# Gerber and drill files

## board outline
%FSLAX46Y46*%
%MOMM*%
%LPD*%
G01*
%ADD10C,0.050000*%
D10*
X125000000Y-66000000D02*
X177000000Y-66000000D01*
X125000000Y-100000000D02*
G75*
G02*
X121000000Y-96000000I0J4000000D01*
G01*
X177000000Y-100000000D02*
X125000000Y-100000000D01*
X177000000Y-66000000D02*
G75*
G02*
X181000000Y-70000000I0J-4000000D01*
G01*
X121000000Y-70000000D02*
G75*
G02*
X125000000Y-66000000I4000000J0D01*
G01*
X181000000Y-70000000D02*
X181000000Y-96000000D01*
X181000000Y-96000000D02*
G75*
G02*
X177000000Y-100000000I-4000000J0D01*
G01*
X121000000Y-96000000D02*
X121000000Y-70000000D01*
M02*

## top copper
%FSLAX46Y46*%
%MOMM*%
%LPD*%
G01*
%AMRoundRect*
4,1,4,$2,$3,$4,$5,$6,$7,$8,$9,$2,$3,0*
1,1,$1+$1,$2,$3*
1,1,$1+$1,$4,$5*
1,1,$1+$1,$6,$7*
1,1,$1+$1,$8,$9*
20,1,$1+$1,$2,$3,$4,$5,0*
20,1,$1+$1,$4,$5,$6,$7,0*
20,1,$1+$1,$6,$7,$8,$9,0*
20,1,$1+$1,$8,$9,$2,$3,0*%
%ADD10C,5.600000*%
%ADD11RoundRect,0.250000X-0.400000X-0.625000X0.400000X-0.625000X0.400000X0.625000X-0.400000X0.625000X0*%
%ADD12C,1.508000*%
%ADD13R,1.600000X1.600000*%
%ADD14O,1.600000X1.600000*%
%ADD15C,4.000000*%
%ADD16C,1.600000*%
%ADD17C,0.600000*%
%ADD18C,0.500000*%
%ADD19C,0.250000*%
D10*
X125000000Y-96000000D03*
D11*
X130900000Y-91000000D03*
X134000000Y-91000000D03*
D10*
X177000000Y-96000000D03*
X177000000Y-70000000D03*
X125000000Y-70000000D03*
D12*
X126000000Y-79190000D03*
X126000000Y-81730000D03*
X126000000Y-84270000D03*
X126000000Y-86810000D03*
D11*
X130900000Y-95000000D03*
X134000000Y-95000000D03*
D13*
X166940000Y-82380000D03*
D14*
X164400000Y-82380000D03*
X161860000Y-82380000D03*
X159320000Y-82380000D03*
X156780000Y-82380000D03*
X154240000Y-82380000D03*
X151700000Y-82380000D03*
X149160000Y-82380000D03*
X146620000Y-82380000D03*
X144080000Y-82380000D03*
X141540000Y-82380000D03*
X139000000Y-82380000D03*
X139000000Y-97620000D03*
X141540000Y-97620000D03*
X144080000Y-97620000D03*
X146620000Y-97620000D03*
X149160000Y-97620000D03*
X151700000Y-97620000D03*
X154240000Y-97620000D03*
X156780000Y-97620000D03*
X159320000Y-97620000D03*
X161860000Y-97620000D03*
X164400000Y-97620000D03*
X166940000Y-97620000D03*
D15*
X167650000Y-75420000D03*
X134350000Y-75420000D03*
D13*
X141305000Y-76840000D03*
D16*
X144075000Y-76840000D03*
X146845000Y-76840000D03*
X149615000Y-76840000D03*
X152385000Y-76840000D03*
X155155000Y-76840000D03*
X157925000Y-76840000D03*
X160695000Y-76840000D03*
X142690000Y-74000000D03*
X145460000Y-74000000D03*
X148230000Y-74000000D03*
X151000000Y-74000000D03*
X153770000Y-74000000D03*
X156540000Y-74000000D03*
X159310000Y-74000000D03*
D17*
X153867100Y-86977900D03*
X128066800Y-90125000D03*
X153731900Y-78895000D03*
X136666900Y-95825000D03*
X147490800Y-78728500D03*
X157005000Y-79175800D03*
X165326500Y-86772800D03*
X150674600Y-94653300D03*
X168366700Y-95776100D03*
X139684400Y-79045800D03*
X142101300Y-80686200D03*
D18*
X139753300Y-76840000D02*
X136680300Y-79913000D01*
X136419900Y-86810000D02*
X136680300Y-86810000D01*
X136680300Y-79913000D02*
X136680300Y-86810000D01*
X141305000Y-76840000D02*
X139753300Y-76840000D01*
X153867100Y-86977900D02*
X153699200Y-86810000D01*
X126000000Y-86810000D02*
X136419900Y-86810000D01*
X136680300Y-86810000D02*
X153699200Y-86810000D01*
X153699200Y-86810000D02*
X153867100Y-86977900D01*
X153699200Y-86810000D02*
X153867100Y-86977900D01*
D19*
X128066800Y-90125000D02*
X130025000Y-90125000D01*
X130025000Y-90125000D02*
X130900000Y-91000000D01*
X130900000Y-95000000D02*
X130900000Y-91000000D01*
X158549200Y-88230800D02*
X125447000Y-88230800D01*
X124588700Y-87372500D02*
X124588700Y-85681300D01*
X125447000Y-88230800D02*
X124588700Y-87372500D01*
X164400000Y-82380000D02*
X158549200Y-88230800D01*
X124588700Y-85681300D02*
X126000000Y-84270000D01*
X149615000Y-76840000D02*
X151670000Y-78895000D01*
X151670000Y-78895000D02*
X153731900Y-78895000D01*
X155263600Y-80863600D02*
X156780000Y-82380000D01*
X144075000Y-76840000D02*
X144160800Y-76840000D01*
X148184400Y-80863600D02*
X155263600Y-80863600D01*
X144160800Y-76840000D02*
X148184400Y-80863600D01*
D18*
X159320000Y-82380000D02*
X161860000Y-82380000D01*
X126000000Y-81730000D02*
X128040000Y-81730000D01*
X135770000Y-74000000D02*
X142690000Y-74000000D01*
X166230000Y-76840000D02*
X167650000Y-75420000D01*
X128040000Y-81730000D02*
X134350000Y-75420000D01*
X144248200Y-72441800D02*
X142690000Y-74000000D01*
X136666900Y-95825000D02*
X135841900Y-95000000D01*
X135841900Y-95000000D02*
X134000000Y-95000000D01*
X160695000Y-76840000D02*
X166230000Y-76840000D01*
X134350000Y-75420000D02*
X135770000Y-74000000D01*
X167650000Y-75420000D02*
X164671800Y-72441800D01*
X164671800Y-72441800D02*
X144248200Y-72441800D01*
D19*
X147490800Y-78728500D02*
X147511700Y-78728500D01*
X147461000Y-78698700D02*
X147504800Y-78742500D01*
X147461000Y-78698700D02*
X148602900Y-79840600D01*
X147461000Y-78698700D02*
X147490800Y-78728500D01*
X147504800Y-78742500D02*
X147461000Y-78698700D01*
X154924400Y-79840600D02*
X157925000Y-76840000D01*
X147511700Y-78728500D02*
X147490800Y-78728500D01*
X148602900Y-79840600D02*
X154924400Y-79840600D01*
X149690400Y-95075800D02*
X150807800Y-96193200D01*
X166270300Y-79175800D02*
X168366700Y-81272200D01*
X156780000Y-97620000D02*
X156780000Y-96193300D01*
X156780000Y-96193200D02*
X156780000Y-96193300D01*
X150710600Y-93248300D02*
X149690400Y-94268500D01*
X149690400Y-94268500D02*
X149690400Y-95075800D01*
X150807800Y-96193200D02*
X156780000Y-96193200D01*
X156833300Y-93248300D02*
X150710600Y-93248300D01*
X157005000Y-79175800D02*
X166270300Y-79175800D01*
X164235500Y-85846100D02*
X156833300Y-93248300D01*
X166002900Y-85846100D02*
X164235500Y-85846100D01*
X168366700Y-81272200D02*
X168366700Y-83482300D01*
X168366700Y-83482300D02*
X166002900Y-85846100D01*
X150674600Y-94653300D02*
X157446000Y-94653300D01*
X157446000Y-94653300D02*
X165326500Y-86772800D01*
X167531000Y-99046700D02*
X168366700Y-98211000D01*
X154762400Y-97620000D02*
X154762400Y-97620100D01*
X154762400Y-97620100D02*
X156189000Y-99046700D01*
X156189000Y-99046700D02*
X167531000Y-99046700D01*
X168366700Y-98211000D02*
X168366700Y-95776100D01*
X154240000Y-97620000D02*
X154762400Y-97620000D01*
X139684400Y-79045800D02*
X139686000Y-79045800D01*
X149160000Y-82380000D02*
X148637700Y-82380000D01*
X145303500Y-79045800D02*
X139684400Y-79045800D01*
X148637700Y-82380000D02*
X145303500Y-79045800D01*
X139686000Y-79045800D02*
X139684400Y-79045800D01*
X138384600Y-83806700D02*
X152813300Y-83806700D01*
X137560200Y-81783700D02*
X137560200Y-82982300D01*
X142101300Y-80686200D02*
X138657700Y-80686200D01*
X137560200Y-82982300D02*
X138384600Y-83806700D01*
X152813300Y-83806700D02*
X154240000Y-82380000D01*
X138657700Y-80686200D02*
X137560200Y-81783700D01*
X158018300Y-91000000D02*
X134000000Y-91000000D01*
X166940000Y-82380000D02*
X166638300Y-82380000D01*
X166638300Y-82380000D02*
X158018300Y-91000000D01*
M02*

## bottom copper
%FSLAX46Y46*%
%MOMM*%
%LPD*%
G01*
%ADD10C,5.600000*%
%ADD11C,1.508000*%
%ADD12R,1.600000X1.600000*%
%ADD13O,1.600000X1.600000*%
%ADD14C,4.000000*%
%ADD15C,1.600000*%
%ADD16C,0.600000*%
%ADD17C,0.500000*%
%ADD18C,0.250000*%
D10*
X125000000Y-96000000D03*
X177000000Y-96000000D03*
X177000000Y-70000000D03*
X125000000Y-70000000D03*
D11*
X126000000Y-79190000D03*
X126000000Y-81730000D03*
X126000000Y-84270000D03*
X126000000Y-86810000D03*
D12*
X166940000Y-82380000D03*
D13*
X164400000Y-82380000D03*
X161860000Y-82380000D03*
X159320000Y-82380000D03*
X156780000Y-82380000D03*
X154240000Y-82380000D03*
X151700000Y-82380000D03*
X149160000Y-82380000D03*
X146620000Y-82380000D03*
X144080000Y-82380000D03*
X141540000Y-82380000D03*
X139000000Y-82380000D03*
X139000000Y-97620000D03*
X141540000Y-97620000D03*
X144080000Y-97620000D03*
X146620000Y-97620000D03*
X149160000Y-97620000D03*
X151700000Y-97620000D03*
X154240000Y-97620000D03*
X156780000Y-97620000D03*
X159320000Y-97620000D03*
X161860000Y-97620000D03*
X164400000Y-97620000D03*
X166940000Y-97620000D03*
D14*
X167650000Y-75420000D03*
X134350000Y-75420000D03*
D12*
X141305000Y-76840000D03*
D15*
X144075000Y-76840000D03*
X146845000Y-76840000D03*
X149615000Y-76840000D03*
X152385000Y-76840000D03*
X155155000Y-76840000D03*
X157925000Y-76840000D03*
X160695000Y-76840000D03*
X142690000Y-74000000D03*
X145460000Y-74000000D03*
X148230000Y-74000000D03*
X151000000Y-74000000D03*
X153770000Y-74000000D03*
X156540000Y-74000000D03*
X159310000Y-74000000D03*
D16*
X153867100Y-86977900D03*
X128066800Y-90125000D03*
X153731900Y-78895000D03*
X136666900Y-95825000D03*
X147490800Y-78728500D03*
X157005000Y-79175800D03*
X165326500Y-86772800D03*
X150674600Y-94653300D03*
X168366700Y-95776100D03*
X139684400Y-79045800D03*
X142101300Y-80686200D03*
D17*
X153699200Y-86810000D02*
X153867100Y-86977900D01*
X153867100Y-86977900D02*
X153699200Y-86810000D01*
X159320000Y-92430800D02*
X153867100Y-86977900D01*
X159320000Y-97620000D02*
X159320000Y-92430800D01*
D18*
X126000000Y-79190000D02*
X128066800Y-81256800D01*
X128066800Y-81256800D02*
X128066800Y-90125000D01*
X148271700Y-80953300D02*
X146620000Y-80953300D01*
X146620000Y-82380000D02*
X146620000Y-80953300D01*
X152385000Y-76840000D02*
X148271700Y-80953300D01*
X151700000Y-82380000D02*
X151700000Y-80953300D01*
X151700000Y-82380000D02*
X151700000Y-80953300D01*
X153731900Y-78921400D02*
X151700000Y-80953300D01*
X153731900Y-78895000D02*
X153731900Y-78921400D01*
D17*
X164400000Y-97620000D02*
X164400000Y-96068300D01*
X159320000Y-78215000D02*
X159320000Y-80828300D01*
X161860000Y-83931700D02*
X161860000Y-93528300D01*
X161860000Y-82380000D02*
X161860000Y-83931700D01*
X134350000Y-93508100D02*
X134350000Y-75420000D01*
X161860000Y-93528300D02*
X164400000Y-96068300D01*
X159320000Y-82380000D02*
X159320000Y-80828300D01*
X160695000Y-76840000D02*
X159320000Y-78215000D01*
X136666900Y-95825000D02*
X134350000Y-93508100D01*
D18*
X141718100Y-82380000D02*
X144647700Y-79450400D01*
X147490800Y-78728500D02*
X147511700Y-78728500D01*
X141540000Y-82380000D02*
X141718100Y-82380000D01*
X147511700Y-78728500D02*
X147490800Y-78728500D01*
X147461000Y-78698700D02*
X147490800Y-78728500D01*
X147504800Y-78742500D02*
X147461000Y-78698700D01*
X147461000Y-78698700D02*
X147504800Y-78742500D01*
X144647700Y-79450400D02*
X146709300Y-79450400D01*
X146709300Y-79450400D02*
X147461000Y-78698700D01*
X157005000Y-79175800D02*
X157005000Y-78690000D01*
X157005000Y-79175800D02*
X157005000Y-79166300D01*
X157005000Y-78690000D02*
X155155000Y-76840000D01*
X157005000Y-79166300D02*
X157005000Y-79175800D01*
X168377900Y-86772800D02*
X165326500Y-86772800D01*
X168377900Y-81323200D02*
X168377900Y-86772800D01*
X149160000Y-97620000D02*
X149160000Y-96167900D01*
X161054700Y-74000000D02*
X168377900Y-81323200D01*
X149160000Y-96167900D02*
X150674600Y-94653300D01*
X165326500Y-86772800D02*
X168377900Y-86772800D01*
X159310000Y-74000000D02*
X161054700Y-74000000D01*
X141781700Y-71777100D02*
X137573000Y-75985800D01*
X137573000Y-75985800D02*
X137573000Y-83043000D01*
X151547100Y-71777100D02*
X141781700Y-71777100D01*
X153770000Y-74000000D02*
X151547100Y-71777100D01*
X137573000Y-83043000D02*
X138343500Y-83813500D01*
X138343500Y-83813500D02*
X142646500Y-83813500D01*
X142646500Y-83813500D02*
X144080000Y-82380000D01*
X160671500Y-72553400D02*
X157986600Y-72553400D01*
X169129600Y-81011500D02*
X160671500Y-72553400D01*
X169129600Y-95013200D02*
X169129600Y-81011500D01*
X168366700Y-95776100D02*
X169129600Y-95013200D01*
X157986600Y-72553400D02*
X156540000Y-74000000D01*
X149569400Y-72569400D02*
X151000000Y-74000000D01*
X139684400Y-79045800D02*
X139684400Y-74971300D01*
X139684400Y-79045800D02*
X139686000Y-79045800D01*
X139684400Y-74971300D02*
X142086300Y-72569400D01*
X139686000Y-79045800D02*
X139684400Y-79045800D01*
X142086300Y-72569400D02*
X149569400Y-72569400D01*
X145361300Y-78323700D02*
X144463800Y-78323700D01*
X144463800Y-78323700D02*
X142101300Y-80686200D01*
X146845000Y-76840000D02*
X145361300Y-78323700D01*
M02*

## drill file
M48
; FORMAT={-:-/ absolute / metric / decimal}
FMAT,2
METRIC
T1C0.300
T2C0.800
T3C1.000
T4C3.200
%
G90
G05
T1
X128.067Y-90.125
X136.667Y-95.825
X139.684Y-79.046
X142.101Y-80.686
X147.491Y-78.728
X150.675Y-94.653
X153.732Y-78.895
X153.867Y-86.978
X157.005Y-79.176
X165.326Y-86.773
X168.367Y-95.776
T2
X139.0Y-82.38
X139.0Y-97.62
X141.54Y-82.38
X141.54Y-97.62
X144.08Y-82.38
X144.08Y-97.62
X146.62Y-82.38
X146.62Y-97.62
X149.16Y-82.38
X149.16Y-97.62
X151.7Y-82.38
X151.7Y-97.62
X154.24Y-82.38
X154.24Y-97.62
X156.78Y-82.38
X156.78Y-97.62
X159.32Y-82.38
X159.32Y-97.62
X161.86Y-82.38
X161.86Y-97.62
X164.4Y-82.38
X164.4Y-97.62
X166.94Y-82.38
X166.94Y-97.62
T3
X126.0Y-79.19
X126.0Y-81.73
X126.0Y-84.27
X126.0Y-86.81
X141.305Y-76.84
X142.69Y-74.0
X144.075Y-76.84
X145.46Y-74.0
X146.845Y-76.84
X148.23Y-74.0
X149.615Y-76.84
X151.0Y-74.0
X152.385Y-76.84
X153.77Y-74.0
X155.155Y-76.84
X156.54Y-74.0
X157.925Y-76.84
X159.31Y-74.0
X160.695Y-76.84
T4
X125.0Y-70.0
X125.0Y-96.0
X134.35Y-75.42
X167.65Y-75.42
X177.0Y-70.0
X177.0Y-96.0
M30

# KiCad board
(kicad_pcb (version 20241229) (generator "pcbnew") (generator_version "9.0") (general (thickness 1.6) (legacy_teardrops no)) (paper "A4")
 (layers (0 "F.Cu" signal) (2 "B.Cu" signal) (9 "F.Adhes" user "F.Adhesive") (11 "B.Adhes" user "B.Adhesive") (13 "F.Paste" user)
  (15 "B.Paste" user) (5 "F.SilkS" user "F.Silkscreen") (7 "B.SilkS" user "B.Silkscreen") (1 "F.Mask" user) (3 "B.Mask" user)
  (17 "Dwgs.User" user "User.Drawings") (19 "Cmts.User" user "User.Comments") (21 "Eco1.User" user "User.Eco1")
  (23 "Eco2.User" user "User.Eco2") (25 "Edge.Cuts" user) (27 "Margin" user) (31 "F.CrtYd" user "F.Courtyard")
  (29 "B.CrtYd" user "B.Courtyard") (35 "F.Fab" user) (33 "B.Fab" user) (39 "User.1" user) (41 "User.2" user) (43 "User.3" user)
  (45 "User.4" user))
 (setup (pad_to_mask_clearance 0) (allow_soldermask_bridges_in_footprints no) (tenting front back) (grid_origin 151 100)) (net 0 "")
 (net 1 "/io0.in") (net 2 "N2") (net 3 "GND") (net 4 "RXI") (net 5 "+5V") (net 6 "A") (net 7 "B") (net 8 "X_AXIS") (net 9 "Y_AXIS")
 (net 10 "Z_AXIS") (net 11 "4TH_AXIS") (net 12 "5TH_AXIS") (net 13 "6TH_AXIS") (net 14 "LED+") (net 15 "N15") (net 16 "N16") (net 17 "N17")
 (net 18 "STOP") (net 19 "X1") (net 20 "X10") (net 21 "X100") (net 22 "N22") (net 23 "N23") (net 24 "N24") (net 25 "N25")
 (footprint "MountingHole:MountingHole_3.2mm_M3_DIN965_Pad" (layer "F.Cu") (at 125 96)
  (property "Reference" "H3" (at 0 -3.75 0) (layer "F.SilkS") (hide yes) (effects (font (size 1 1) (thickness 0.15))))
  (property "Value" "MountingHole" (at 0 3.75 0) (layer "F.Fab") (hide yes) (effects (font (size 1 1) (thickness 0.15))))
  (pad "1" thru_hole circle (at 0 0) (size 5.6 5.6) (drill 3.2) (layers "*.Cu" "*.Mask") (remove_unused_layers no) (zone_connect 2)))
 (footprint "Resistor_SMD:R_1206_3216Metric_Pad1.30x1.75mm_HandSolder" (layer "F.Cu") (at 132.45 91)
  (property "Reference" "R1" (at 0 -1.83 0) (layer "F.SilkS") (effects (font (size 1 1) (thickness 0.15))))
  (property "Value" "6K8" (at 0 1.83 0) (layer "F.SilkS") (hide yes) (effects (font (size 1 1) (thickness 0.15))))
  (pad "1" smd roundrect (at -1.55 0) (size 1.3 1.75) (layers "F.Cu" "F.Mask" "F.Paste") (roundrect_rratio 0.192308) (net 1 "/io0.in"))
  (pad "2" smd roundrect (at 1.55 0) (size 1.3 1.75) (layers "F.Cu" "F.Mask" "F.Paste") (roundrect_rratio 0.192308) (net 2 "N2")))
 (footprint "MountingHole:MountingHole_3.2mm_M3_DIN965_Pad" (layer "F.Cu") (at 177 96)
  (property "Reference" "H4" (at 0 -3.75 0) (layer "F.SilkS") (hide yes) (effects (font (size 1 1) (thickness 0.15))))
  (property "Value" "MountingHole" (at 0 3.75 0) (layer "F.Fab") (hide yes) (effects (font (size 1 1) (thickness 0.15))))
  (pad "1" thru_hole circle (at 0 0) (size 5.6 5.6) (drill 3.2) (layers "*.Cu" "*.Mask") (remove_unused_layers no) (zone_connect 2)))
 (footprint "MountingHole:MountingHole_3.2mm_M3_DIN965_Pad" (layer "F.Cu") (at 177 70)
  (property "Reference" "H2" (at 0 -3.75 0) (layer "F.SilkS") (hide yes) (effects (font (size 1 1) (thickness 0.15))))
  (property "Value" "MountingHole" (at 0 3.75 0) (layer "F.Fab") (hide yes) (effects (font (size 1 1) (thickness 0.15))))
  (pad "1" thru_hole circle (at 0 0) (size 5.6 5.6) (drill 3.2) (layers "*.Cu" "*.Mask") (remove_unused_layers no) (zone_connect 2)))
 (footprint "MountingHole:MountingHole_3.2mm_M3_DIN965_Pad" (layer "F.Cu") (at 125 70)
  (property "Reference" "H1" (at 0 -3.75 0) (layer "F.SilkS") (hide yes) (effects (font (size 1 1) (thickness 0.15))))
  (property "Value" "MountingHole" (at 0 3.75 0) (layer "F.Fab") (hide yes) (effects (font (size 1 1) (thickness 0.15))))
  (pad "1" thru_hole circle (at 0 0) (size 5.6 5.6) (drill 3.2) (layers "*.Cu" "*.Mask") (remove_unused_layers no) (zone_connect 2)))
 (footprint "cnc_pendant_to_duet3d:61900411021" (layer "F.Cu") (at 122.65 83 -90)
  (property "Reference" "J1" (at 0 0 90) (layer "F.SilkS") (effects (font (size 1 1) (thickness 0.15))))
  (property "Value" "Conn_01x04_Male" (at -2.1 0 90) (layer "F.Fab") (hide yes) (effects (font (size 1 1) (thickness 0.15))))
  (pad "1" thru_hole circle (at -3.81 -3.35 270) (size 1.508 1.508) (drill 1) (layers "*.Cu" "*.Mask") (remove_unused_layers no)
   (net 1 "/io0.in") (solder_mask_margin 0.102))
  (pad "2" thru_hole circle (at -1.27 -3.35 270) (size 1.508 1.508) (drill 1) (layers "*.Cu" "*.Mask") (remove_unused_layers no)
   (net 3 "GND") (solder_mask_margin 0.102))
  (pad "3" thru_hole circle (at 1.27 -3.35 270) (size 1.508 1.508) (drill 1) (layers "*.Cu" "*.Mask") (remove_unused_layers no)
   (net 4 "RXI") (solder_mask_margin 0.102))
  (pad "4" thru_hole circle (at 3.81 -3.35 270) (size 1.508 1.508) (drill 1) (layers "*.Cu" "*.Mask") (remove_unused_layers no)
   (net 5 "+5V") (solder_mask_margin 0.102)))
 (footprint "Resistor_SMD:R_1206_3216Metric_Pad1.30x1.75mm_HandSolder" (layer "F.Cu") (at 132.45 95)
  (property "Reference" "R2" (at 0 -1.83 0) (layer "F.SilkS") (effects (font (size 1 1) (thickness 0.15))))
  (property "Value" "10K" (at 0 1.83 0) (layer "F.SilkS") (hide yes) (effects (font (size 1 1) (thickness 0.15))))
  (pad "1" smd roundrect (at -1.55 0) (size 1.3 1.75) (layers "F.Cu" "F.Mask" "F.Paste") (roundrect_rratio 0.192308) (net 1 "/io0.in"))
  (pad "2" smd roundrect (at 1.55 0) (size 1.3 1.75) (layers "F.Cu" "F.Mask" "F.Paste") (roundrect_rratio 0.192308) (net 3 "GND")))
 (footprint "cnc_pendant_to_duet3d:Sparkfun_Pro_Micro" (layer "F.Cu") (at 139 97.62 90)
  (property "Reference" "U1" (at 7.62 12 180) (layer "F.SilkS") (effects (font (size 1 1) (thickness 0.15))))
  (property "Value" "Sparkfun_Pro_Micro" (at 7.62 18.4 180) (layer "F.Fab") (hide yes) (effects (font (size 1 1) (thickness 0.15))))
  (pad "1" thru_hole rect (at 15.24 27.94 90) (size 1.6 1.6) (drill 0.8) (layers "*.Cu" "*.Mask") (remove_unused_layers no) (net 2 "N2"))
  (pad "2" thru_hole oval (at 15.24 25.4 90) (size 1.6 1.6) (drill 0.8) (layers "*.Cu" "*.Mask") (remove_unused_layers no) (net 4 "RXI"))
  (pad "3" thru_hole oval (at 15.24 22.86 90) (size 1.6 1.6) (drill 0.8) (layers "*.Cu" "*.Mask") (remove_unused_layers no) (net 3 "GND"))
  (pad "4" thru_hole oval (at 15.24 20.32 90) (size 1.6 1.6) (drill 0.8) (layers "*.Cu" "*.Mask") (remove_unused_layers no) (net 3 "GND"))
  (pad "5" thru_hole oval (at 15.24 17.78 90) (size 1.6 1.6) (drill 0.8) (layers "*.Cu" "*.Mask") (remove_unused_layers no) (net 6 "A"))
  (pad "6" thru_hole oval (at 15.24 15.24 90) (size 1.6 1.6) (drill 0.8) (layers "*.Cu" "*.Mask") (remove_unused_layers no) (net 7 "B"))
  (pad "7" thru_hole oval (at 15.24 12.7 90) (size 1.6 1.6) (drill 0.8) (layers "*.Cu" "*.Mask") (remove_unused_layers no) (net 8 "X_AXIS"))
  (pad "8" thru_hole oval (at 15.24 10.16 90) (size 1.6 1.6) (drill 0.8) (layers "*.Cu" "*.Mask") (remove_unused_layers no) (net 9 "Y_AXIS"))
  (pad "9" thru_hole oval (at 15.24 7.62 90) (size 1.6 1.6) (drill 0.8) (layers "*.Cu" "*.Mask") (remove_unused_layers no) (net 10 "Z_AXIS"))
  (pad "10" thru_hole oval (at 15.24 5.08 90) (size 1.6 1.6) (drill 0.8) (layers "*.Cu" "*.Mask") (remove_unused_layers no)
   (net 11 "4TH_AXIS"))
  (pad "11" thru_hole oval (at 15.24 2.54 90) (size 1.6 1.6) (drill 0.8) (layers "*.Cu" "*.Mask") (remove_unused_layers no)
   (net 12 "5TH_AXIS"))
  (pad "12" thru_hole oval (at 15.24 0 90) (size 1.6 1.6) (drill 0.8) (layers "*.Cu" "*.Mask") (remove_unused_layers no) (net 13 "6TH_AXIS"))
  (pad "13" thru_hole oval (at 0 0 90) (size 1.6 1.6) (drill 0.8) (layers "*.Cu" "*.Mask") (remove_unused_layers no) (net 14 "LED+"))
  (pad "14" thru_hole oval (at 0 2.54 90) (size 1.6 1.6) (drill 0.8) (layers "*.Cu" "*.Mask") (remove_unused_layers no) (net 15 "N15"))
  (pad "15" thru_hole oval (at 0 5.08 90) (size 1.6 1.6) (drill 0.8) (layers "*.Cu" "*.Mask") (remove_unused_layers no) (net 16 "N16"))
  (pad "16" thru_hole oval (at 0 7.62 90) (size 1.6 1.6) (drill 0.8) (layers "*.Cu" "*.Mask") (remove_unused_layers no) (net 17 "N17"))
  (pad "17" thru_hole oval (at 0 10.16 90) (size 1.6 1.6) (drill 0.8) (layers "*.Cu" "*.Mask") (remove_unused_layers no) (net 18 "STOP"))
  (pad "18" thru_hole oval (at 0 12.7 90) (size 1.6 1.6) (drill 0.8) (layers "*.Cu" "*.Mask") (remove_unused_layers no) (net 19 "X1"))
  (pad "19" thru_hole oval (at 0 15.24 90) (size 1.6 1.6) (drill 0.8) (layers "*.Cu" "*.Mask") (remove_unused_layers no) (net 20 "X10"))
  (pad "20" thru_hole oval (at 0 17.78 90) (size 1.6 1.6) (drill 0.8) (layers "*.Cu" "*.Mask") (remove_unused_layers no) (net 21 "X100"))
  (pad "21" thru_hole oval (at 0 20.32 90) (size 1.6 1.6) (drill 0.8) (layers "*.Cu" "*.Mask") (remove_unused_layers no) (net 5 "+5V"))
  (pad "22" thru_hole oval (at 0 22.86 90) (size 1.6 1.6) (drill 0.8) (layers "*.Cu" "*.Mask") (remove_unused_layers no) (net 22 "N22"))
  (pad "23" thru_hole oval (at 0 25.4 90) (size 1.6 1.6) (drill 0.8) (layers "*.Cu" "*.Mask") (remove_unused_layers no) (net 3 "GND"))
  (pad "24" thru_hole oval (at 0 27.94 90) (size 1.6 1.6) (drill 0.8) (layers "*.Cu" "*.Mask") (remove_unused_layers no) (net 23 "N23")))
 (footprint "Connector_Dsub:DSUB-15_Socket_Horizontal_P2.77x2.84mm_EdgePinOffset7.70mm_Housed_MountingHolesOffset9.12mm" (layer "F.Cu")
  (at 141.305 76.84 180)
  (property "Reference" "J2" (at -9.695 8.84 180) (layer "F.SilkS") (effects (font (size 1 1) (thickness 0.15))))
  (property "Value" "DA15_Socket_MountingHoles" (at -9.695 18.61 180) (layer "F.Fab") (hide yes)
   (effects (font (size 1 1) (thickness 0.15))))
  (pad "0" thru_hole circle (at -26.345 1.42 180) (size 4 4) (drill 3.2) (layers "*.Cu" "*.Mask") (remove_unused_layers no) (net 3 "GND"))
  (pad "0" thru_hole circle (at 6.955 1.42 180) (size 4 4) (drill 3.2) (layers "*.Cu" "*.Mask") (remove_unused_layers no) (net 3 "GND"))
  (pad "1" thru_hole rect (at 0 0 180) (size 1.6 1.6) (drill 1) (layers "*.Cu" "*.Mask") (remove_unused_layers no) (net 5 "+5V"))
  (pad "2" thru_hole circle (at -2.77 0 180) (size 1.6 1.6) (drill 1) (layers "*.Cu" "*.Mask") (remove_unused_layers no) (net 6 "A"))
  (pad "3" thru_hole circle (at -5.54 0 180) (size 1.6 1.6) (drill 1) (layers "*.Cu" "*.Mask") (remove_unused_layers no) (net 7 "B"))
  (pad "4" thru_hole circle (at -8.31 0 180) (size 1.6 1.6) (drill 1) (layers "*.Cu" "*.Mask") (remove_unused_layers no) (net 8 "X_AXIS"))
  (pad "5" thru_hole circle (at -11.08 0 180) (size 1.6 1.6) (drill 1) (layers "*.Cu" "*.Mask") (remove_unused_layers no) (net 10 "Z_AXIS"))
  (pad "6" thru_hole circle (at -13.85 0 180) (size 1.6 1.6) (drill 1) (layers "*.Cu" "*.Mask") (remove_unused_layers no) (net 21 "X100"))
  (pad "7" thru_hole circle (at -16.62 0 180) (size 1.6 1.6) (drill 1) (layers "*.Cu" "*.Mask") (remove_unused_layers no)
   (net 12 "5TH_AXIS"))
  (pad "8" thru_hole circle (at -19.39 0 180) (size 1.6 1.6) (drill 1) (layers "*.Cu" "*.Mask") (remove_unused_layers no) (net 3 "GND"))
  (pad "9" thru_hole circle (at -1.385 2.84 180) (size 1.6 1.6) (drill 1) (layers "*.Cu" "*.Mask") (remove_unused_layers no) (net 3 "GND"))
  (pad "10" thru_hole circle (at -4.155 2.84 180) (size 1.6 1.6) (drill 1) (layers "*.Cu" "*.Mask") (remove_unused_layers no) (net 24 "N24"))
  (pad "11" thru_hole circle (at -6.925 2.84 180) (size 1.6 1.6) (drill 1) (layers "*.Cu" "*.Mask") (remove_unused_layers no) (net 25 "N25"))
  (pad "12" thru_hole circle (at -9.695 2.84 180) (size 1.6 1.6) (drill 1) (layers "*.Cu" "*.Mask") (remove_unused_layers no)
   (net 9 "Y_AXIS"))
  (pad "13" thru_hole circle (at -12.465 2.84 180) (size 1.6 1.6) (drill 1) (layers "*.Cu" "*.Mask") (remove_unused_layers no)
   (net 11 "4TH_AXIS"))
  (pad "14" thru_hole circle (at -15.235 2.84 180) (size 1.6 1.6) (drill 1) (layers "*.Cu" "*.Mask") (remove_unused_layers no)
   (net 20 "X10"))
  (pad "15" thru_hole circle (at -18.005 2.84 180) (size 1.6 1.6) (drill 1) (layers "*.Cu" "*.Mask") (remove_unused_layers no)
   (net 18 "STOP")))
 (gr_line (start 125 66) (end 177 66) (stroke (width 0.05) (type default)) (layer "Edge.Cuts"))
 (gr_arc (start 125 100) (mid 122.171573 98.828427) (end 121 96) (stroke (width 0.05) (type default)) (layer "Edge.Cuts"))
 (gr_line (start 177 100) (end 125 100) (stroke (width 0.05) (type default)) (layer "Edge.Cuts"))
 (gr_arc (start 177 66) (mid 179.828427 67.171573) (end 181 70) (stroke (width 0.05) (type default)) (layer "Edge.Cuts"))
 (gr_arc (start 121 70) (mid 122.171573 67.171573) (end 125 66) (stroke (width 0.05) (type default)) (layer "Edge.Cuts"))
 (gr_line (start 181 70) (end 181 96) (stroke (width 0.05) (type default)) (layer "Edge.Cuts"))
 (gr_arc (start 181 96) (mid 179.828427 98.828427) (end 177 100) (stroke (width 0.05) (type default)) (layer "Edge.Cuts"))
 (gr_line (start 121 96) (end 121 70) (stroke (width 0.05) (type default)) (layer "Edge.Cuts"))
 (segment (start 139.7533 76.84) (end 136.6803 79.913) (width 0.5) (layer "F.Cu") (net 5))
 (segment (start 136.4199 86.81) (end 136.6803 86.81) (width 0.5) (layer "F.Cu") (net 5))
 (segment (start 136.6803 79.913) (end 136.6803 86.81) (width 0.5) (layer "F.Cu") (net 5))
 (segment (start 141.305 76.84) (end 139.7533 76.84) (width 0.5) (layer "F.Cu") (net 5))
 (segment (start 153.8671 86.9779) (end 153.6992 86.81) (width 0.5) (layer "F.Cu") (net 5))
 (segment (start 126 86.81) (end 136.4199 86.81) (width 0.5) (layer "F.Cu") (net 5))
 (segment (start 136.6803 86.81) (end 153.6992 86.81) (width 0.5) (layer "F.Cu") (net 5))
 (segment (start 153.6992 86.81) (end 153.8671 86.9779) (width 0.5) (layer "F.Cu") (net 5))
 (segment (start 153.6992 86.81) (end 153.8671 86.9779) (width 0.5) (layer "F.Cu") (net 5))
 (via (at 153.8671 86.9779) (size 0.6) (drill 0.3) (layers "F.Cu" "B.Cu") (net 5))
 (segment (start 153.6992 86.81) (end 153.8671 86.9779) (width 0.5) (layer "B.Cu") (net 5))
 (segment (start 153.8671 86.9779) (end 153.6992 86.81) (width 0.5) (layer "B.Cu") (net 5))
 (segment (start 159.32 92.4308) (end 153.8671 86.9779) (width 0.5) (layer "B.Cu") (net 5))
 (segment (start 159.32 97.62) (end 159.32 92.4308) (width 0.5) (layer "B.Cu") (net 5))
 (segment (start 128.0668 90.125) (end 130.025 90.125) (width 0.25) (layer "F.Cu") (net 1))
 (segment (start 130.025 90.125) (end 130.9 91) (width 0.25) (layer "F.Cu") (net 1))
 (segment (start 130.9 95) (end 130.9 91) (width 0.25) (layer "F.Cu") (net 1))
 (via (at 128.0668 90.125) (size 0.6) (drill 0.3) (layers "F.Cu" "B.Cu") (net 1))
 (segment (start 126 79.19) (end 128.0668 81.2568) (width 0.25) (layer "B.Cu") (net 1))
 (segment (start 128.0668 81.2568) (end 128.0668 90.125) (width 0.25) (layer "B.Cu") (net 1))
 (segment (start 158.5492 88.2308) (end 125.447 88.2308) (width 0.25) (layer "F.Cu") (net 4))
 (segment (start 124.5887 87.3725) (end 124.5887 85.6813) (width 0.25) (layer "F.Cu") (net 4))
 (segment (start 125.447 88.2308) (end 124.5887 87.3725) (width 0.25) (layer "F.Cu") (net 4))
 (segment (start 164.4 82.38) (end 158.5492 88.2308) (width 0.25) (layer "F.Cu") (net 4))
 (segment (start 124.5887 85.6813) (end 126 84.27) (width 0.25) (layer "F.Cu") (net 4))
 (segment (start 148.2717 80.9533) (end 146.62 80.9533) (width 0.25) (layer "B.Cu") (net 10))
 (segment (start 146.62 82.38) (end 146.62 80.9533) (width 0.25) (layer "B.Cu") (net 10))
 (segment (start 152.385 76.84) (end 148.2717 80.9533) (width 0.25) (layer "B.Cu") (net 10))
 (segment (start 149.615 76.84) (end 151.67 78.895) (width 0.25) (layer "F.Cu") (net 8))
 (segment (start 151.67 78.895) (end 153.7319 78.895) (width 0.25) (layer "F.Cu") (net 8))
 (via (at 153.7319 78.895) (size 0.6) (drill 0.3) (layers "F.Cu" "B.Cu") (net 8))
 (segment (start 151.7 82.38) (end 151.7 80.9533) (width 0.25) (layer "B.Cu") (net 8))
 (segment (start 151.7 82.38) (end 151.7 80.9533) (width 0.25) (layer "B.Cu") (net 8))
 (segment (start 153.7319 78.9214) (end 151.7 80.9533) (width 0.25) (layer "B.Cu") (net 8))
 (segment (start 153.7319 78.895) (end 153.7319 78.9214) (width 0.25) (layer "B.Cu") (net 8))
 (segment (start 155.2636 80.8636) (end 156.78 82.38) (width 0.25) (layer "F.Cu") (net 6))
 (segment (start 144.075 76.84) (end 144.1608 76.84) (width 0.25) (layer "F.Cu") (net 6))
 (segment (start 148.1844 80.8636) (end 155.2636 80.8636) (width 0.25) (layer "F.Cu") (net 6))
 (segment (start 144.1608 76.84) (end 148.1844 80.8636) (width 0.25) (layer "F.Cu") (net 6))
 (segment (start 159.32 82.38) (end 161.86 82.38) (width 0.5) (layer "F.Cu") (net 3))
 (segment (start 126 81.73) (end 128.04 81.73) (width 0.5) (layer "F.Cu") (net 3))
 (segment (start 135.77 74) (end 142.69 74) (width 0.5) (layer "F.Cu") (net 3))
 (segment (start 166.23 76.84) (end 167.65 75.42) (width 0.5) (layer "F.Cu") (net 3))
 (segment (start 128.04 81.73) (end 134.35 75.42) (width 0.5) (layer "F.Cu") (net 3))
 (segment (start 144.2482 72.4418) (end 142.69 74) (width 0.5) (layer "F.Cu") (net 3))
 (segment (start 136.6669 95.825) (end 135.8419 95) (width 0.5) (layer "F.Cu") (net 3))
 (segment (start 135.8419 95) (end 134 95) (width 0.5) (layer "F.Cu") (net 3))
 (segment (start 160.695 76.84) (end 166.23 76.84) (width 0.5) (layer "F.Cu") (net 3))
 (segment (start 134.35 75.42) (end 135.77 74) (width 0.5) (layer "F.Cu") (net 3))
 (segment (start 167.65 75.42) (end 164.6718 72.4418) (width 0.5) (layer "F.Cu") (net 3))
 (segment (start 164.6718 72.4418) (end 144.2482 72.4418) (width 0.5) (layer "F.Cu") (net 3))
 (via (at 136.6669 95.825) (size 0.6) (drill 0.3) (layers "F.Cu" "B.Cu") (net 3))
 (segment (start 164.4 97.62) (end 164.4 96.0683) (width 0.5) (layer "B.Cu") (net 3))
 (segment (start 159.32 78.215) (end 159.32 80.8283) (width 0.5) (layer "B.Cu") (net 3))
 (segment (start 161.86 83.9317) (end 161.86 93.5283) (width 0.5) (layer "B.Cu") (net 3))
 (segment (start 161.86 82.38) (end 161.86 83.9317) (width 0.5) (layer "B.Cu") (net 3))
 (segment (start 134.35 93.5081) (end 134.35 75.42) (width 0.5) (layer "B.Cu") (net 3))
 (segment (start 161.86 93.5283) (end 164.4 96.0683) (width 0.5) (layer "B.Cu") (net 3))
 (segment (start 159.32 82.38) (end 159.32 80.8283) (width 0.5) (layer "B.Cu") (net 3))
 (segment (start 160.695 76.84) (end 159.32 78.215) (width 0.5) (layer "B.Cu") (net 3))
 (segment (start 136.6669 95.825) (end 134.35 93.5081) (width 0.5) (layer "B.Cu") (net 3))
 (segment (start 147.4908 78.7285) (end 147.5117 78.7285) (width 0.25) (layer "F.Cu") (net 12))
 (segment (start 147.461 78.6987) (end 147.5048 78.7425) (width 0.25) (layer "F.Cu") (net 12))
 (segment (start 147.461 78.6987) (end 148.6029 79.8406) (width 0.25) (layer "F.Cu") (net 12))
 (segment (start 147.461 78.6987) (end 147.4908 78.7285) (width 0.25) (layer "F.Cu") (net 12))
 (segment (start 147.5048 78.7425) (end 147.461 78.6987) (width 0.25) (layer "F.Cu") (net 12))
 (segment (start 154.9244 79.8406) (end 157.925 76.84) (width 0.25) (layer "F.Cu") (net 12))
 (segment (start 147.5117 78.7285) (end 147.4908 78.7285) (width 0.25) (layer "F.Cu") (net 12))
 (segment (start 148.6029 79.8406) (end 154.9244 79.8406) (width 0.25) (layer "F.Cu") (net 12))
 (via (at 147.4908 78.7285) (size 0.6) (drill 0.3) (layers "F.Cu" "B.Cu") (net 12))
 (segment (start 141.7181 82.38) (end 144.6477 79.4504) (width 0.25) (layer "B.Cu") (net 12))
 (segment (start 147.4908 78.7285) (end 147.5117 78.7285) (width 0.25) (layer "B.Cu") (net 12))
 (segment (start 141.54 82.38) (end 141.7181 82.38) (width 0.25) (layer "B.Cu") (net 12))
 (segment (start 147.5117 78.7285) (end 147.4908 78.7285) (width 0.25) (layer "B.Cu") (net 12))
 (segment (start 147.461 78.6987) (end 147.4908 78.7285) (width 0.25) (layer "B.Cu") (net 12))
 (segment (start 147.5048 78.7425) (end 147.461 78.6987) (width 0.25) (layer "B.Cu") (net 12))
 (segment (start 147.461 78.6987) (end 147.5048 78.7425) (width 0.25) (layer "B.Cu") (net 12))
 (segment (start 144.6477 79.4504) (end 146.7093 79.4504) (width 0.25) (layer "B.Cu") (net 12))
 (segment (start 146.7093 79.4504) (end 147.461 78.6987) (width 0.25) (layer "B.Cu") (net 12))
 (segment (start 149.6904 95.0758) (end 150.8078 96.1932) (width 0.25) (layer "F.Cu") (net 21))
 (segment (start 166.2703 79.1758) (end 168.3667 81.2722) (width 0.25) (layer "F.Cu") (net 21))
 (segment (start 156.78 97.62) (end 156.78 96.1933) (width 0.25) (layer "F.Cu") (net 21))
 (segment (start 156.78 96.1932) (end 156.78 96.1933) (width 0.25) (layer "F.Cu") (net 21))
 (segment (start 150.7106 93.2483) (end 149.6904 94.2685) (width 0.25) (layer "F.Cu") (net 21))
 (segment (start 149.6904 94.2685) (end 149.6904 95.0758) (width 0.25) (layer "F.Cu") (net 21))
 (segment (start 150.8078 96.1932) (end 156.78 96.1932) (width 0.25) (layer "F.Cu") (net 21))
 (segment (start 156.8333 93.2483) (end 150.7106 93.2483) (width 0.25) (layer "F.Cu") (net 21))
 (segment (start 157.005 79.1758) (end 166.2703 79.1758) (width 0.25) (layer "F.Cu") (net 21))
 (segment (start 164.2355 85.8461) (end 156.8333 93.2483) (width 0.25) (layer "F.Cu") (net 21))
 (segment (start 166.0029 85.8461) (end 164.2355 85.8461) (width 0.25) (layer "F.Cu") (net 21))
 (segment (start 168.3667 81.2722) (end 168.3667 83.4823) (width 0.25) (layer "F.Cu") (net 21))
 (segment (start 168.3667 83.4823) (end 166.0029 85.8461) (width 0.25) (layer "F.Cu") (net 21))
 (via (at 157.005 79.1758) (size 0.6) (drill 0.3) (layers "F.Cu" "B.Cu") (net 21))
 (segment (start 157.005 79.1758) (end 157.005 78.69) (width 0.25) (layer "B.Cu") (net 21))
 (segment (start 157.005 79.1758) (end 157.005 79.1663) (width 0.25) (layer "B.Cu") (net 21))
 (segment (start 157.005 78.69) (end 155.155 76.84) (width 0.25) (layer "B.Cu") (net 21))
 (segment (start 157.005 79.1663) (end 157.005 79.1758) (width 0.25) (layer "B.Cu") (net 21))
 (segment (start 150.6746 94.6533) (end 157.446 94.6533) (width 0.25) (layer "F.Cu") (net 18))
 (segment (start 157.446 94.6533) (end 165.3265 86.7728) (width 0.25) (layer "F.Cu") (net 18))
 (via (at 165.3265 86.7728) (size 0.6) (drill 0.3) (layers "F.Cu" "B.Cu") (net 18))
 (via (at 150.6746 94.6533) (size 0.6) (drill 0.3) (layers "F.Cu" "B.Cu") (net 18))
 (segment (start 168.3779 86.7728) (end 165.3265 86.7728) (width 0.25) (layer "B.Cu") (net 18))
 (segment (start 168.3779 81.3232) (end 168.3779 86.7728) (width 0.25) (layer "B.Cu") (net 18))
 (segment (start 149.16 97.62) (end 149.16 96.1679) (width 0.25) (layer "B.Cu") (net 18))
 (segment (start 161.0547 74) (end 168.3779 81.3232) (width 0.25) (layer "B.Cu") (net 18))
 (segment (start 149.16 96.1679) (end 150.6746 94.6533) (width 0.25) (layer "B.Cu") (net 18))
 (segment (start 165.3265 86.7728) (end 168.3779 86.7728) (width 0.25) (layer "B.Cu") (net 18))
 (segment (start 159.31 74) (end 161.0547 74) (width 0.25) (layer "B.Cu") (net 18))
 (segment (start 141.7817 71.7771) (end 137.573 75.9858) (width 0.25) (layer "B.Cu") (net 11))
 (segment (start 137.573 75.9858) (end 137.573 83.043) (width 0.25) (layer "B.Cu") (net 11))
 (segment (start 151.5471 71.7771) (end 141.7817 71.7771) (width 0.25) (layer "B.Cu") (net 11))
 (segment (start 153.77 74) (end 151.5471 71.7771) (width 0.25) (layer "B.Cu") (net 11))
 (segment (start 137.573 83.043) (end 138.3435 83.8135) (width 0.25) (layer "B.Cu") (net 11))
 (segment (start 138.3435 83.8135) (end 142.6465 83.8135) (width 0.25) (layer "B.Cu") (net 11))
 (segment (start 142.6465 83.8135) (end 144.08 82.38) (width 0.25) (layer "B.Cu") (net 11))
 (segment (start 167.531 99.0467) (end 168.3667 98.211) (width 0.25) (layer "F.Cu") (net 20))
 (segment (start 154.7624 97.62) (end 154.7624 97.6201) (width 0.25) (layer "F.Cu") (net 20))
 (segment (start 154.7624 97.6201) (end 156.189 99.0467) (width 0.25) (layer "F.Cu") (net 20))
 (segment (start 156.189 99.0467) (end 167.531 99.0467) (width 0.25) (layer "F.Cu") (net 20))
 (segment (start 168.3667 98.211) (end 168.3667 95.7761) (width 0.25) (layer "F.Cu") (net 20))
 (segment (start 154.24 97.62) (end 154.7624 97.62) (width 0.25) (layer "F.Cu") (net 20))
 (via (at 168.3667 95.7761) (size 0.6) (drill 0.3) (layers "F.Cu" "B.Cu") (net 20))
 (segment (start 160.6715 72.5534) (end 157.9866 72.5534) (width 0.25) (layer "B.Cu") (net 20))
 (segment (start 169.1296 81.0115) (end 160.6715 72.5534) (width 0.25) (layer "B.Cu") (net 20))
 (segment (start 169.1296 95.0132) (end 169.1296 81.0115) (width 0.25) (layer "B.Cu") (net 20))
 (segment (start 168.3667 95.7761) (end 169.1296 95.0132) (width 0.25) (layer "B.Cu") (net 20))
 (segment (start 157.9866 72.5534) (end 156.54 74) (width 0.25) (layer "B.Cu") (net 20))
 (segment (start 139.6844 79.0458) (end 139.686 79.0458) (width 0.25) (layer "F.Cu") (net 9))
 (segment (start 149.16 82.38) (end 148.6377 82.38) (width 0.25) (layer "F.Cu") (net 9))
 (segment (start 145.3035 79.0458) (end 139.6844 79.0458) (width 0.25) (layer "F.Cu") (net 9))
 (segment (start 148.6377 82.38) (end 145.3035 79.0458) (width 0.25) (layer "F.Cu") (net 9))
 (segment (start 139.686 79.0458) (end 139.6844 79.0458) (width 0.25) (layer "F.Cu") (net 9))
 (via (at 139.6844 79.0458) (size 0.6) (drill 0.3) (layers "F.Cu" "B.Cu") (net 9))
 (segment (start 149.5694 72.5694) (end 151 74) (width 0.25) (layer "B.Cu") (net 9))
 (segment (start 139.6844 79.0458) (end 139.6844 74.9713) (width 0.25) (layer "B.Cu") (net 9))
 (segment (start 139.6844 79.0458) (end 139.686 79.0458) (width 0.25) (layer "B.Cu") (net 9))
 (segment (start 139.6844 74.9713) (end 142.0863 72.5694) (width 0.25) (layer "B.Cu") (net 9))
 (segment (start 139.686 79.0458) (end 139.6844 79.0458) (width 0.25) (layer "B.Cu") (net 9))
 (segment (start 142.0863 72.5694) (end 149.5694 72.5694) (width 0.25) (layer "B.Cu") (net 9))
 (segment (start 138.3846 83.8067) (end 152.8133 83.8067) (width 0.25) (layer "F.Cu") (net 7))
 (segment (start 137.5602 81.7837) (end 137.5602 82.9823) (width 0.25) (layer "F.Cu") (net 7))
 (segment (start 142.1013 80.6862) (end 138.6577 80.6862) (width 0.25) (layer "F.Cu") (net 7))
 (segment (start 137.5602 82.9823) (end 138.3846 83.8067) (width 0.25) (layer "F.Cu") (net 7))
 (segment (start 152.8133 83.8067) (end 154.24 82.38) (width 0.25) (layer "F.Cu") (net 7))
 (segment (start 138.6577 80.6862) (end 137.5602 81.7837) (width 0.25) (layer "F.Cu") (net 7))
 (via (at 142.1013 80.6862) (size 0.6) (drill 0.3) (layers "F.Cu" "B.Cu") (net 7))
 (segment (start 145.3613 78.3237) (end 144.4638 78.3237) (width 0.25) (layer "B.Cu") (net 7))
 (segment (start 144.4638 78.3237) (end 142.1013 80.6862) (width 0.25) (layer "B.Cu") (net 7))
 (segment (start 146.845 76.84) (end 145.3613 78.3237) (width 0.25) (layer "B.Cu") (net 7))
 (segment (start 158.0183 91) (end 134 91) (width 0.25) (layer "F.Cu") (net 2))
 (segment (start 166.94 82.38) (end 166.6383 82.38) (width 0.25) (layer "F.Cu") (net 2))
 (segment (start 166.6383 82.38) (end 158.0183 91) (width 0.25) (layer "F.Cu") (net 2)))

